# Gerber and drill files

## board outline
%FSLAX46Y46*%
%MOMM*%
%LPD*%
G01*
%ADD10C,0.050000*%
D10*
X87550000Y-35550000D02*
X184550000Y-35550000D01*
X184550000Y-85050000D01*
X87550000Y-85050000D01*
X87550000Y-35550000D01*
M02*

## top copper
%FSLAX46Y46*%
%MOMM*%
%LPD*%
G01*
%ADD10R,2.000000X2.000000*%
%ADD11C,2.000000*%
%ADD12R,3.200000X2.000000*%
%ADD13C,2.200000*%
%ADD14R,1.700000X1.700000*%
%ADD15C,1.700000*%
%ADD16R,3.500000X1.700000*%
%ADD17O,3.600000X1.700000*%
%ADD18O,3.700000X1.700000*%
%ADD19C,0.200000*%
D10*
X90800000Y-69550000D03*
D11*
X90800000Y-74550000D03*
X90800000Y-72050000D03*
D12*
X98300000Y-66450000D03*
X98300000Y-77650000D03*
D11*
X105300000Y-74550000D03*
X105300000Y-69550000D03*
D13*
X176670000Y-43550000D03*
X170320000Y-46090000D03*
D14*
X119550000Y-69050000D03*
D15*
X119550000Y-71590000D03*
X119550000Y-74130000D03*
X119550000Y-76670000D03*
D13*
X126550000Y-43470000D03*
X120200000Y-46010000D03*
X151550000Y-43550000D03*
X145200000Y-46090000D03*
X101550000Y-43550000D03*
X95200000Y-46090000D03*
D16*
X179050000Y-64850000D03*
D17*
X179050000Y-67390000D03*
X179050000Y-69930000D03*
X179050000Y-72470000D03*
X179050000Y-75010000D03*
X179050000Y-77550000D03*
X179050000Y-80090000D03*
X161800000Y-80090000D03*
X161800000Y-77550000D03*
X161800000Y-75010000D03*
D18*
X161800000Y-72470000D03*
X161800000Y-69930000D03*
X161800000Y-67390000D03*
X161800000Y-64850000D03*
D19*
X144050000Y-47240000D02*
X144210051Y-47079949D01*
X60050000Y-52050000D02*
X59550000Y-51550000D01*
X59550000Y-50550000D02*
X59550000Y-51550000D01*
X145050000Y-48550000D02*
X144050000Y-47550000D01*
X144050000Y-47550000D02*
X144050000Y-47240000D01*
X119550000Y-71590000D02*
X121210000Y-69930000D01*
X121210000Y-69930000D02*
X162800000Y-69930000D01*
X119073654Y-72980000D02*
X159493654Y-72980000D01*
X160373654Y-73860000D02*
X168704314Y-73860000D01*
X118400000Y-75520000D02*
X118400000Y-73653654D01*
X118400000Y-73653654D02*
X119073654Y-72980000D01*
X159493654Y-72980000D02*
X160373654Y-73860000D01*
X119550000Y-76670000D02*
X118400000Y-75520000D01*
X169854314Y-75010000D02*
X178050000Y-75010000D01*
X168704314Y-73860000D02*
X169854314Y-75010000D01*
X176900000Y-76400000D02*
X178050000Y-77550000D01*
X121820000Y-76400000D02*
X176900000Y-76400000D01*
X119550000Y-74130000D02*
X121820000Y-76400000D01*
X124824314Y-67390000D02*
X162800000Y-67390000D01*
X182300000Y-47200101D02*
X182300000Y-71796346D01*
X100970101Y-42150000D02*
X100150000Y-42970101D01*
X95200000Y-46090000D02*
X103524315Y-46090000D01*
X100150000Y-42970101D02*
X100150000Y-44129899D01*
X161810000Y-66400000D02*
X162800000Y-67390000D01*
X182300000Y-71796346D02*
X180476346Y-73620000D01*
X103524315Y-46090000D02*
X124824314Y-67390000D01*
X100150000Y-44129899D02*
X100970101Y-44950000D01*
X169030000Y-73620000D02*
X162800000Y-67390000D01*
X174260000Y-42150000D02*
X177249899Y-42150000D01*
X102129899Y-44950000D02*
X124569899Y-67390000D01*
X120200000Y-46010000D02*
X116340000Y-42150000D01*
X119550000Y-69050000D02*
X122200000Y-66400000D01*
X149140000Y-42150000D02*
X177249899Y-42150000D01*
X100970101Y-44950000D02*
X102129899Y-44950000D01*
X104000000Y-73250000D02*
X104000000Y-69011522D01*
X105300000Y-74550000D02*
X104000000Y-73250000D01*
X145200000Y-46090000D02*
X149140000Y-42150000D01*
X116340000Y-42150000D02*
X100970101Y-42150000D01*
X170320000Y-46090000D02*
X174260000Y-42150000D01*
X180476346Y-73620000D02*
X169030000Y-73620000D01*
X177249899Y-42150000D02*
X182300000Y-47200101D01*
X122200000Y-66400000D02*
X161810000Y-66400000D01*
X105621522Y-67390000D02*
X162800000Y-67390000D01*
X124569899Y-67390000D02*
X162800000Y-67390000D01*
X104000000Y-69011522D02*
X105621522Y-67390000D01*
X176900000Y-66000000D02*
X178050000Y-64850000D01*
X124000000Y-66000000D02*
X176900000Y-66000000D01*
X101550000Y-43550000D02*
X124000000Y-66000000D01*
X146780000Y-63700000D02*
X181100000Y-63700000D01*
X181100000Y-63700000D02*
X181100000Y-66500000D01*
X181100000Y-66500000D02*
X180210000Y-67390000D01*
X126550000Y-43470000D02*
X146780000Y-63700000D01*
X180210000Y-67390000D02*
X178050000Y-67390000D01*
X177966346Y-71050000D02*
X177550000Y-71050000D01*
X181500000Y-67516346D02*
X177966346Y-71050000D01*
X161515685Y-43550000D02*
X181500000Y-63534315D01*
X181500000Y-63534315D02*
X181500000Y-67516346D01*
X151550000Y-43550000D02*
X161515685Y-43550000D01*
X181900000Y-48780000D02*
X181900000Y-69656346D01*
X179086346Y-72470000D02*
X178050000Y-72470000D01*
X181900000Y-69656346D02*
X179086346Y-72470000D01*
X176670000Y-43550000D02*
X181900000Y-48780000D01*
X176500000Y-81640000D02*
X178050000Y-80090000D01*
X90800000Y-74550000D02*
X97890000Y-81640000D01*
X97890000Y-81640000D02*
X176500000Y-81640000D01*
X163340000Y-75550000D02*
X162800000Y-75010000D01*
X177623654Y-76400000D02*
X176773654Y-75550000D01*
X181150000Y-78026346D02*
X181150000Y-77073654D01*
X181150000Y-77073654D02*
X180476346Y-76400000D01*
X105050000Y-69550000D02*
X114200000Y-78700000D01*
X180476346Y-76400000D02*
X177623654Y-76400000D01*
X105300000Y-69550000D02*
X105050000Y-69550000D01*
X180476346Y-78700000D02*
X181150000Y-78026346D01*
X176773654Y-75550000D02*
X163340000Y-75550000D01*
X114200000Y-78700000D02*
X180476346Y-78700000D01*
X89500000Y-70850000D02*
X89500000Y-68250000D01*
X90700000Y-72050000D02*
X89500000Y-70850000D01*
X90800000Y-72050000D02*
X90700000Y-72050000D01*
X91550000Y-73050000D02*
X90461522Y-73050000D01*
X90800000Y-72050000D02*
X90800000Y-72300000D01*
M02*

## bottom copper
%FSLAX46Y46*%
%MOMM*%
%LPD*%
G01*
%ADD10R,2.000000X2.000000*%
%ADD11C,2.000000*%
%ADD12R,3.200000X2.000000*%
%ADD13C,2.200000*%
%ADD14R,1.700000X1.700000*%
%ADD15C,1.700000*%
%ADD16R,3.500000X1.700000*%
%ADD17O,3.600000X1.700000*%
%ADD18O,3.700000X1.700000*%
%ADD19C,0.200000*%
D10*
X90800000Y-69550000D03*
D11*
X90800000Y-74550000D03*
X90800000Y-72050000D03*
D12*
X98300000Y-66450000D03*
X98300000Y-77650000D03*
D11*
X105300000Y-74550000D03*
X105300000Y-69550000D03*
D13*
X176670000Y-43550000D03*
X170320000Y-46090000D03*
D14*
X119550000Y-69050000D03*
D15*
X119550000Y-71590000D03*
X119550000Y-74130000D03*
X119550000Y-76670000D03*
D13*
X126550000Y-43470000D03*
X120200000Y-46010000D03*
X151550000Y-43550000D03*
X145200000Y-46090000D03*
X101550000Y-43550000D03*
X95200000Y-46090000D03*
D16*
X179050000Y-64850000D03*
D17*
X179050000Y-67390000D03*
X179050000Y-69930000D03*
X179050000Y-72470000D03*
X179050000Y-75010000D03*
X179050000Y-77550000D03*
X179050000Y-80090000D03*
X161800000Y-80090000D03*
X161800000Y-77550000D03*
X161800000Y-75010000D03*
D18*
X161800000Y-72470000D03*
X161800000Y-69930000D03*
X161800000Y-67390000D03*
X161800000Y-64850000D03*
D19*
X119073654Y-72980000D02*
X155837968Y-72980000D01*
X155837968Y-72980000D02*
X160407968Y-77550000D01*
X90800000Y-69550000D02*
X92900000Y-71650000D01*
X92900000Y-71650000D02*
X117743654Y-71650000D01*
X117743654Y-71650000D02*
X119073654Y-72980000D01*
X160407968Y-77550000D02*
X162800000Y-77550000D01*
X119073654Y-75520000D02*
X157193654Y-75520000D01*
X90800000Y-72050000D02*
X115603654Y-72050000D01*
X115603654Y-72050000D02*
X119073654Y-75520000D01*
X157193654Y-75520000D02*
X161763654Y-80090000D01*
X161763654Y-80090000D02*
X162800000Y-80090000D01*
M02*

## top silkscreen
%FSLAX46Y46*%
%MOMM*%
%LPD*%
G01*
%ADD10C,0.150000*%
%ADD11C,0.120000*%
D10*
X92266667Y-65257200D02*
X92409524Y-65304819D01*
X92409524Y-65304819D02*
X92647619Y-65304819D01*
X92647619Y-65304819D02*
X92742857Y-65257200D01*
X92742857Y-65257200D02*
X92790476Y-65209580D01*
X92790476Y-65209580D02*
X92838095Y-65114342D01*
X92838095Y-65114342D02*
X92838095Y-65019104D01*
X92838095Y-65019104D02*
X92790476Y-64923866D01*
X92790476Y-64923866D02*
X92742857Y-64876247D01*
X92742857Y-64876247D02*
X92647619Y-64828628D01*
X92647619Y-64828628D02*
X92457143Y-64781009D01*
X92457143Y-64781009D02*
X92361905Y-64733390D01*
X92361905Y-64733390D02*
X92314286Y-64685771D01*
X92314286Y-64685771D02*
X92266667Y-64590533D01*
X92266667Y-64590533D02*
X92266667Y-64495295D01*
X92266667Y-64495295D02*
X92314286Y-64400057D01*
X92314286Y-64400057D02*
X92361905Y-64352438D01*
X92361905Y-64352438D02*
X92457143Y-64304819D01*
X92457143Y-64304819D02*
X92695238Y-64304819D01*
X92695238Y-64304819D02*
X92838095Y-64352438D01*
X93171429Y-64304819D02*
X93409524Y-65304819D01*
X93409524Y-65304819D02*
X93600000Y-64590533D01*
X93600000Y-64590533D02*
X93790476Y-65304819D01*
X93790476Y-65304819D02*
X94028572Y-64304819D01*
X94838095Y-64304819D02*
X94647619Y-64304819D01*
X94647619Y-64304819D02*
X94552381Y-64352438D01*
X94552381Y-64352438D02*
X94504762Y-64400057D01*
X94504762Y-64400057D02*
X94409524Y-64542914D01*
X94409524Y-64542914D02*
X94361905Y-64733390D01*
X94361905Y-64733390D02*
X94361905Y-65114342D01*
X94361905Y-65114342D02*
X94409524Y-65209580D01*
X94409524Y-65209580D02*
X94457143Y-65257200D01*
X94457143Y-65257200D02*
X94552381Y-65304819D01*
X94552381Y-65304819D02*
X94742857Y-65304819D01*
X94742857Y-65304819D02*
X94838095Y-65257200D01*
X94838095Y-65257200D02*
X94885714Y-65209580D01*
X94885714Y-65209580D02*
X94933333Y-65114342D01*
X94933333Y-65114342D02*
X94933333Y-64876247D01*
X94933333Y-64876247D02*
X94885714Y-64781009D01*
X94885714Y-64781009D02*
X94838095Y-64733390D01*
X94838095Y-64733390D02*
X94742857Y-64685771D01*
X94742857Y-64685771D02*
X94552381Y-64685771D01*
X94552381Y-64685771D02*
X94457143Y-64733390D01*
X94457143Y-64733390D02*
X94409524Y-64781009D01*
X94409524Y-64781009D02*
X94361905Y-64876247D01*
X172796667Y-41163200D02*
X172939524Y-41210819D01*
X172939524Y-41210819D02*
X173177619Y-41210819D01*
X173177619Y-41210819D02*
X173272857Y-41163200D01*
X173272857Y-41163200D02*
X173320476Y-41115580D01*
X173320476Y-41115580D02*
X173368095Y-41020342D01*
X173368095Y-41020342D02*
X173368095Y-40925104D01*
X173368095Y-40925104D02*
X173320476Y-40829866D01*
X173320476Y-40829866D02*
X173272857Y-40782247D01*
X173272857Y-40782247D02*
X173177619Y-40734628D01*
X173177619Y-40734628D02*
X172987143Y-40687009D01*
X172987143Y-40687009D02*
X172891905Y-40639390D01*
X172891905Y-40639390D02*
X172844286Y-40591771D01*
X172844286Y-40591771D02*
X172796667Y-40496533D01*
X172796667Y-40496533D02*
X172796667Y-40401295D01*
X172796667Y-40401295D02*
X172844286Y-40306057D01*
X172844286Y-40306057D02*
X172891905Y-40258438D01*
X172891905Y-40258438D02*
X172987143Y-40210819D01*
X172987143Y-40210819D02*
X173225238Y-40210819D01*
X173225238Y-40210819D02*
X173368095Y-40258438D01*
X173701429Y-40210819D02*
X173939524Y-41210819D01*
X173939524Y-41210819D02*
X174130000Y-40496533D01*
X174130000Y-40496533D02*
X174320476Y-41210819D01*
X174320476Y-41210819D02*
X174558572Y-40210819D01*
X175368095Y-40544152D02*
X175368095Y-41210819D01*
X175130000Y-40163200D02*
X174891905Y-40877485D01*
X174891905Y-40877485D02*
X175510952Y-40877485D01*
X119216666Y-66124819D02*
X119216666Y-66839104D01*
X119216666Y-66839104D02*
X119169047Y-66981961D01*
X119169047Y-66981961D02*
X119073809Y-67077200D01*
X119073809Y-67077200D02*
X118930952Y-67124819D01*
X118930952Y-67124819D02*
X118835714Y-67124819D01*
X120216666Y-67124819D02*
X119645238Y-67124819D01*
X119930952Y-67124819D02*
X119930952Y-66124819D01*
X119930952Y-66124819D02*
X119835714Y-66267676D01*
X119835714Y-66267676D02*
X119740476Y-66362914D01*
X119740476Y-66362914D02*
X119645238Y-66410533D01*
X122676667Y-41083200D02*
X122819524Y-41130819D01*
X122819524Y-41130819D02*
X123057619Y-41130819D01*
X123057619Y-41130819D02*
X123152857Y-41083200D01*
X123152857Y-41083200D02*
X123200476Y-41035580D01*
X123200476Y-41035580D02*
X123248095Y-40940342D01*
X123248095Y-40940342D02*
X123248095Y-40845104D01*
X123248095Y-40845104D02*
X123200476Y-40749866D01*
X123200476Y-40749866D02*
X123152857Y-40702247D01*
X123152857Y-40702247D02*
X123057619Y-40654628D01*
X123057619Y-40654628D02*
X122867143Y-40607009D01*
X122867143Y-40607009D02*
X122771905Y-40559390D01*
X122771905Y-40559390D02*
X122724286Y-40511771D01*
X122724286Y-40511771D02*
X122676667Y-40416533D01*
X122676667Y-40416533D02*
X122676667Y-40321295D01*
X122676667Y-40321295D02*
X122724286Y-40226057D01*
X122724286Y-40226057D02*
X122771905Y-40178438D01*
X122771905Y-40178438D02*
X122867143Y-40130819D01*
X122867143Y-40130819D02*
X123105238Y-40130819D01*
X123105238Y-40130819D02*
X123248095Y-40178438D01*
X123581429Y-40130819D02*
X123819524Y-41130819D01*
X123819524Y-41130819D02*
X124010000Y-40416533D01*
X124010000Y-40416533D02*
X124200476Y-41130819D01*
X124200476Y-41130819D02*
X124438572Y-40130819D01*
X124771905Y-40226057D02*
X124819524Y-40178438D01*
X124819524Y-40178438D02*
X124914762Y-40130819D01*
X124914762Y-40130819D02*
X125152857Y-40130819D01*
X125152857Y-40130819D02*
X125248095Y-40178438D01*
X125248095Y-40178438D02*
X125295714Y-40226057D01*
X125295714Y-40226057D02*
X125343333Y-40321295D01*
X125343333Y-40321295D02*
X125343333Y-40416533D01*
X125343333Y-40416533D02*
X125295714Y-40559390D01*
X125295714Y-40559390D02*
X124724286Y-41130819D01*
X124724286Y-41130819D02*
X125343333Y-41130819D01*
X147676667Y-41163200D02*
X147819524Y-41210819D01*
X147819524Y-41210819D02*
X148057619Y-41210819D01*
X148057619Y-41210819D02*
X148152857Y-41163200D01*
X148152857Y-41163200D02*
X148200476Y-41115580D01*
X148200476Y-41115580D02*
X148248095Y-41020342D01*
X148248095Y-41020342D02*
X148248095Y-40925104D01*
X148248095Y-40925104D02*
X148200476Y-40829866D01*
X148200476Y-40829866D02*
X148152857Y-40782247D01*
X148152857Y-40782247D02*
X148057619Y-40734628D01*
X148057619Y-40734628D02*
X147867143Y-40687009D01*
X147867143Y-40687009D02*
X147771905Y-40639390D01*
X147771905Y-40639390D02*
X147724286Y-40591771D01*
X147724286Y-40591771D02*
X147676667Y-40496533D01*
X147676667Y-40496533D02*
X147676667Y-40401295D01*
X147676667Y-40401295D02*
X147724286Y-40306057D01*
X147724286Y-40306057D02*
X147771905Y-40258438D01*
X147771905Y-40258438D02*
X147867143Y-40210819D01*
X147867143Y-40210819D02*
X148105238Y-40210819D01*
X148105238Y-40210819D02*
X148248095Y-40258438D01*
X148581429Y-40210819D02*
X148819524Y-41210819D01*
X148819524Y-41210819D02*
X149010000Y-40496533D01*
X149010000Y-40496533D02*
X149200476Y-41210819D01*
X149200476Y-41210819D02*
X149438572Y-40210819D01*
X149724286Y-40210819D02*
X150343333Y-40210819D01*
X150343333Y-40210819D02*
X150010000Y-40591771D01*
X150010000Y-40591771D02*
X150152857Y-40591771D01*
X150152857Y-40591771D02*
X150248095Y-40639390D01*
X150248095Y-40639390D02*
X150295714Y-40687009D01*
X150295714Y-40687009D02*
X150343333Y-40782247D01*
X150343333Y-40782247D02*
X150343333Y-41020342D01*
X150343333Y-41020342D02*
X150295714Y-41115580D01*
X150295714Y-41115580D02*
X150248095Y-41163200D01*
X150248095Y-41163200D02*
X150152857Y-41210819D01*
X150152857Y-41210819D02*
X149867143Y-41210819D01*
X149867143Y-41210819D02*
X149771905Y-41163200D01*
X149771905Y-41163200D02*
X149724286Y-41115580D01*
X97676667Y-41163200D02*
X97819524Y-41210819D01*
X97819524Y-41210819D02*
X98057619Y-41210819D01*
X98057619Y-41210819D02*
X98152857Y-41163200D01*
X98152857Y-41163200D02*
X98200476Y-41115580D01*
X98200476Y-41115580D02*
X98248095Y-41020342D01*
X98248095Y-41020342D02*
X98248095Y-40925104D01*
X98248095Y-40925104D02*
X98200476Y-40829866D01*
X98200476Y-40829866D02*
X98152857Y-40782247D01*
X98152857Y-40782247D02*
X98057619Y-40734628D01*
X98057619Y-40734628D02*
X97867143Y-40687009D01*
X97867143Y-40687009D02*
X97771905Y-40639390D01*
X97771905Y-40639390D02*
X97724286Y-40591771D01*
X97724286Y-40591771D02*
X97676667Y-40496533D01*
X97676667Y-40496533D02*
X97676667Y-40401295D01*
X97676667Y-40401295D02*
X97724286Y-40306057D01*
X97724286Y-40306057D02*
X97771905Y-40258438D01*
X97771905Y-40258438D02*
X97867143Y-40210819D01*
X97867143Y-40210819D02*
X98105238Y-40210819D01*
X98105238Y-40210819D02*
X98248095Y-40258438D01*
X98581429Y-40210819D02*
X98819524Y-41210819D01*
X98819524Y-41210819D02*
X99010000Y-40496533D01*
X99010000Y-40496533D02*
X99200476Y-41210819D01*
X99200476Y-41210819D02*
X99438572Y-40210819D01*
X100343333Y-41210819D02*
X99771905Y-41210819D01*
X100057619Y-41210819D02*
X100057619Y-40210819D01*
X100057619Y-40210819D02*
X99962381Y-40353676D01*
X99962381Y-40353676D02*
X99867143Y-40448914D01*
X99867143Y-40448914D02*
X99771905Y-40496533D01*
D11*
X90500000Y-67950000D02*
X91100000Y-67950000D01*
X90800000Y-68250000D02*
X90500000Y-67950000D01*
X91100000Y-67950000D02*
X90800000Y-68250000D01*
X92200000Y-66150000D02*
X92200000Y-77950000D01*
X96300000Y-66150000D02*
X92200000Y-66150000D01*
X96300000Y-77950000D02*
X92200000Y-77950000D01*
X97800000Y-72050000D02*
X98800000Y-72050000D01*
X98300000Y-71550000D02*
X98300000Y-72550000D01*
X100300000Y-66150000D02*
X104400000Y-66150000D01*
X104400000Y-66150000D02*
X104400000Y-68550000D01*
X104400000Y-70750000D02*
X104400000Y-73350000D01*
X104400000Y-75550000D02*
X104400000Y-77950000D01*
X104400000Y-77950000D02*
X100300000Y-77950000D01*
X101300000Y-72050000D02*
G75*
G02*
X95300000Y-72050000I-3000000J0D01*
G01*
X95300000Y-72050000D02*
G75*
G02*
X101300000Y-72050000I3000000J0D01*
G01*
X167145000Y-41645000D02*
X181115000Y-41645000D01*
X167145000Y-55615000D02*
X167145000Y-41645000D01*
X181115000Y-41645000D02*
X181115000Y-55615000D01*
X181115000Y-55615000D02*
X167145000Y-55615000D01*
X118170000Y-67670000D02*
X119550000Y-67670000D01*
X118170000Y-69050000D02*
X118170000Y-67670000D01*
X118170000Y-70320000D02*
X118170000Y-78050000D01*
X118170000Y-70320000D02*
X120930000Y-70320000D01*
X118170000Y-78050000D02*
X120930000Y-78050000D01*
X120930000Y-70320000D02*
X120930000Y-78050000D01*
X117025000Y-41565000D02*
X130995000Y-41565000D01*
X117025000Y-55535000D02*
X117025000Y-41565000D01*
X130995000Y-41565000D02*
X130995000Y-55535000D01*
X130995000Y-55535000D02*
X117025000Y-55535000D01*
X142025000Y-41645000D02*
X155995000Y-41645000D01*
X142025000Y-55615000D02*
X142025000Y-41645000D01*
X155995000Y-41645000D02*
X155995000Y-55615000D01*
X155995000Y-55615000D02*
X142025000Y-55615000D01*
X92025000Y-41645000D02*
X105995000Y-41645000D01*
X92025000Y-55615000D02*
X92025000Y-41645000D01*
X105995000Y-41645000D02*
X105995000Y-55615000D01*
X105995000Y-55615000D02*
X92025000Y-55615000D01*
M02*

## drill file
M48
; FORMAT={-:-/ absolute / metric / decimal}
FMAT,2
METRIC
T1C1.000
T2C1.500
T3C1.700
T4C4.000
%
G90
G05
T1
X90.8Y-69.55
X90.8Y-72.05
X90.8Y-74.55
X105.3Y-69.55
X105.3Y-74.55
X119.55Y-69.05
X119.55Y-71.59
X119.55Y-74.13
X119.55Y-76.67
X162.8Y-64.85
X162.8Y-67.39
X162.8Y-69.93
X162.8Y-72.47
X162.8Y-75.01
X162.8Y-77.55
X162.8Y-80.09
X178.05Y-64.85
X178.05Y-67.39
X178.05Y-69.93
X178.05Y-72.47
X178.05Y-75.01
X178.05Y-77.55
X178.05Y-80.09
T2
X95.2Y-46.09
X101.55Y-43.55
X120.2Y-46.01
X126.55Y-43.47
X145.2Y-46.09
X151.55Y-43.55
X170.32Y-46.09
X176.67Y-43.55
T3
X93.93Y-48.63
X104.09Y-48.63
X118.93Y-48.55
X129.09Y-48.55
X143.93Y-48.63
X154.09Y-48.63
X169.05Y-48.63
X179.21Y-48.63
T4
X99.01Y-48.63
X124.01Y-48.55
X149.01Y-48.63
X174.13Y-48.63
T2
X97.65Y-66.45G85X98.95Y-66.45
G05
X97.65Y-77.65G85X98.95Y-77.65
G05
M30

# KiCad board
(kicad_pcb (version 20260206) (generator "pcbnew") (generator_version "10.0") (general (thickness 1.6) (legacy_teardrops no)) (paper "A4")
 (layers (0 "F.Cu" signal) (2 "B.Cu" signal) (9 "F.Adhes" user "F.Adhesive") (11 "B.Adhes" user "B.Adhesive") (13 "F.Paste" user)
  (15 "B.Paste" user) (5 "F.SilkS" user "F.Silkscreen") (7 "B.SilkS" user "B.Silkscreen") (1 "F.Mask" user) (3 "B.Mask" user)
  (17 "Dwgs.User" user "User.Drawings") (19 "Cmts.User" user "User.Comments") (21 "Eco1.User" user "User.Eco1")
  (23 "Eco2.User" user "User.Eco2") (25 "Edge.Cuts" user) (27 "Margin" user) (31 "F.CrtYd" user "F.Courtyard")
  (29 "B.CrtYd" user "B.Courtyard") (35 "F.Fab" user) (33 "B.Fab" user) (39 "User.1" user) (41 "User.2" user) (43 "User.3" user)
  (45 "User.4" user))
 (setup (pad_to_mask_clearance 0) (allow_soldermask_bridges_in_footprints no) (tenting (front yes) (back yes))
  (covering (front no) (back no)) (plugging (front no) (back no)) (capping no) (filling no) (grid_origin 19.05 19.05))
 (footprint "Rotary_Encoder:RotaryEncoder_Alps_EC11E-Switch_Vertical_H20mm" (layer "F.Cu") (at 90.8 69.55)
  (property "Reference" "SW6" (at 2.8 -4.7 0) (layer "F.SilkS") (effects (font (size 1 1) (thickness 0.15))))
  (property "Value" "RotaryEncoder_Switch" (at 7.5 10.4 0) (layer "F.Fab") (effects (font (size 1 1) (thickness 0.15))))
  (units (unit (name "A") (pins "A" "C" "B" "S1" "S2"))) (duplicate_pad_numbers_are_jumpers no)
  (fp_line (start -0.3 -1.6) (end 0.3 -1.6) (stroke (width 0.12) (type solid)) (layer "F.SilkS"))
  (fp_line (start 0 -1.3) (end -0.3 -1.6) (stroke (width 0.12) (type solid)) (layer "F.SilkS"))
  (fp_line (start 0.3 -1.6) (end 0 -1.3) (stroke (width 0.12) (type solid)) (layer "F.SilkS"))
  (fp_line (start 1.4 -3.4) (end 1.4 8.4) (stroke (width 0.12) (type solid)) (layer "F.SilkS"))
  (fp_line (start 5.5 -3.4) (end 1.4 -3.4) (stroke (width 0.12) (type solid)) (layer "F.SilkS"))
  (fp_line (start 5.5 8.4) (end 1.4 8.4) (stroke (width 0.12) (type solid)) (layer "F.SilkS"))
  (fp_line (start 7 2.5) (end 8 2.5) (stroke (width 0.12) (type solid)) (layer "F.SilkS"))
  (fp_line (start 7.5 2) (end 7.5 3) (stroke (width 0.12) (type solid)) (layer "F.SilkS"))
  (fp_line (start 9.5 -3.4) (end 13.6 -3.4) (stroke (width 0.12) (type solid)) (layer "F.SilkS"))
  (fp_line (start 13.6 -3.4) (end 13.6 -1) (stroke (width 0.12) (type solid)) (layer "F.SilkS"))
  (fp_line (start 13.6 1.2) (end 13.6 3.8) (stroke (width 0.12) (type solid)) (layer "F.SilkS"))
  (fp_line (start 13.6 6) (end 13.6 8.4) (stroke (width 0.12) (type solid)) (layer "F.SilkS"))
  (fp_line (start 13.6 8.4) (end 9.5 8.4) (stroke (width 0.12) (type solid)) (layer "F.SilkS"))
  (fp_circle (center 7.5 2.5) (end 10.5 2.5) (stroke (width 0.12) (type solid)) (fill no) (layer "F.SilkS"))
  (pad "A" thru_hole rect (at 0 0) (size 2 2) (drill 1) (layers "*.Cu" "*.Mask") (remove_unused_layers no) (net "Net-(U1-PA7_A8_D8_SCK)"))
  (pad "B" thru_hole circle (at 0 5) (size 2 2) (drill 1) (layers "*.Cu" "*.Mask") (remove_unused_layers no) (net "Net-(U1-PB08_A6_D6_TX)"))
  (pad "C" thru_hole circle (at 0 2.5) (size 2 2) (drill 1) (layers "*.Cu" "*.Mask") (remove_unused_layers no)
   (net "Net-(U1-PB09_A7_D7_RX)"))
  (pad "MP" thru_hole rect (at 7.5 -3.1) (size 3.2 2) (drill oval 2.8 1.5) (layers "*.Cu" "*.Mask") (remove_unused_layers no))
  (pad "MP" thru_hole rect (at 7.5 8.1) (size 3.2 2) (drill oval 2.8 1.5) (layers "*.Cu" "*.Mask") (remove_unused_layers no))
  (pad "S1" thru_hole circle (at 14.5 5) (size 2 2) (drill 1) (layers "*.Cu" "*.Mask") (remove_unused_layers no) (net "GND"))
  (pad "S2" thru_hole circle (at 14.5 0) (size 2 2) (drill 1) (layers "*.Cu" "*.Mask") (remove_unused_layers no)
   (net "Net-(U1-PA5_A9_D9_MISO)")))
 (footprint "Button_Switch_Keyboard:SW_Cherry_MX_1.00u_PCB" (layer "F.Cu") (at 176.67 43.55)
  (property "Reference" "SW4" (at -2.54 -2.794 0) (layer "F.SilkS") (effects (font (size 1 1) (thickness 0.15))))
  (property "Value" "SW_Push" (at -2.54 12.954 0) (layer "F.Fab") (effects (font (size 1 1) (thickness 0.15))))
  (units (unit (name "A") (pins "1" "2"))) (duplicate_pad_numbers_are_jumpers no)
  (fp_line (start -9.525 -1.905) (end 4.445 -1.905) (stroke (width 0.12) (type solid)) (layer "F.SilkS"))
  (fp_line (start -9.525 12.065) (end -9.525 -1.905) (stroke (width 0.12) (type solid)) (layer "F.SilkS"))
  (fp_line (start 4.445 -1.905) (end 4.445 12.065) (stroke (width 0.12) (type solid)) (layer "F.SilkS"))
  (fp_line (start 4.445 12.065) (end -9.525 12.065) (stroke (width 0.12) (type solid)) (layer "F.SilkS"))
  (pad "" np_thru_hole circle (at -7.62 5.08) (size 1.7 1.7) (drill 1.7) (layers "*.Cu" "*.Mask"))
  (pad "" np_thru_hole circle (at -2.54 5.08) (size 4 4) (drill 4) (layers "*.Cu" "*.Mask"))
  (pad "" np_thru_hole circle (at 2.54 5.08) (size 1.7 1.7) (drill 1.7) (layers "*.Cu" "*.Mask"))
  (pad "1" thru_hole circle (at 0 0) (size 2.2 2.2) (drill 1.5) (layers "*.Cu" "*.Mask") (remove_unused_layers no)
   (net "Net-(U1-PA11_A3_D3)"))
  (pad "2" thru_hole circle (at -6.35 2.54) (size 2.2 2.2) (drill 1.5) (layers "*.Cu" "*.Mask") (remove_unused_layers no) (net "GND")))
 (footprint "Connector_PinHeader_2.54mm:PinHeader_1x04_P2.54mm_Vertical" (layer "F.Cu") (at 119.55 69.05)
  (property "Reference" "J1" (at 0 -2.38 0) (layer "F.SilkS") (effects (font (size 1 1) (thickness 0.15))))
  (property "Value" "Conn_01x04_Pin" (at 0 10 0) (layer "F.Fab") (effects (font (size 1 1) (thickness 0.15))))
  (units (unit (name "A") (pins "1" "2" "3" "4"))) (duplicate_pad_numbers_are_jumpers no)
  (fp_line (start -1.38 -1.38) (end 0 -1.38) (stroke (width 0.12) (type solid)) (layer "F.SilkS"))
  (fp_line (start -1.38 0) (end -1.38 -1.38) (stroke (width 0.12) (type solid)) (layer "F.SilkS"))
  (fp_line (start -1.38 1.27) (end -1.38 9) (stroke (width 0.12) (type solid)) (layer "F.SilkS"))
  (fp_line (start -1.38 1.27) (end 1.38 1.27) (stroke (width 0.12) (type solid)) (layer "F.SilkS"))
  (fp_line (start -1.38 9) (end 1.38 9) (stroke (width 0.12) (type solid)) (layer "F.SilkS"))
  (fp_line (start 1.38 1.27) (end 1.38 9) (stroke (width 0.12) (type solid)) (layer "F.SilkS"))
  (pad "1" thru_hole rect (at 0 0) (size 1.7 1.7) (drill 1) (layers "*.Cu" "*.Mask") (remove_unused_layers no) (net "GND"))
  (pad "2" thru_hole circle (at 0 2.54) (size 1.7 1.7) (drill 1) (layers "*.Cu" "*.Mask") (remove_unused_layers no) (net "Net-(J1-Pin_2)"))
  (pad "3" thru_hole circle (at 0 5.08) (size 1.7 1.7) (drill 1) (layers "*.Cu" "*.Mask") (remove_unused_layers no) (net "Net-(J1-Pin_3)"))
  (pad "4" thru_hole circle (at 0 7.62) (size 1.7 1.7) (drill 1) (layers "*.Cu" "*.Mask") (remove_unused_layers no) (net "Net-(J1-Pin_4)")))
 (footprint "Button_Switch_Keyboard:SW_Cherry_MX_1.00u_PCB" (layer "F.Cu") (at 126.55 43.47)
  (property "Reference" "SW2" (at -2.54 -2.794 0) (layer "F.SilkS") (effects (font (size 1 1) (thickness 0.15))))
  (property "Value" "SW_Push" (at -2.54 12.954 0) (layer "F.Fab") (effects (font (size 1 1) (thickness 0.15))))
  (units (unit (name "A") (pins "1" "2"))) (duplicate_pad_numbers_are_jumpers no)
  (fp_line (start -9.525 -1.905) (end 4.445 -1.905) (stroke (width 0.12) (type solid)) (layer "F.SilkS"))
  (fp_line (start -9.525 12.065) (end -9.525 -1.905) (stroke (width 0.12) (type solid)) (layer "F.SilkS"))
  (fp_line (start 4.445 -1.905) (end 4.445 12.065) (stroke (width 0.12) (type solid)) (layer "F.SilkS"))
  (fp_line (start 4.445 12.065) (end -9.525 12.065) (stroke (width 0.12) (type solid)) (layer "F.SilkS"))
  (pad "" np_thru_hole circle (at -7.62 5.08) (size 1.7 1.7) (drill 1.7) (layers "*.Cu" "*.Mask"))
  (pad "" np_thru_hole circle (at -2.54 5.08) (size 4 4) (drill 4) (layers "*.Cu" "*.Mask"))
  (pad "" np_thru_hole circle (at 2.54 5.08) (size 1.7 1.7) (drill 1.7) (layers "*.Cu" "*.Mask"))
  (pad "1" thru_hole circle (at 0 0) (size 2.2 2.2) (drill 1.5) (layers "*.Cu" "*.Mask") (remove_unused_layers no)
   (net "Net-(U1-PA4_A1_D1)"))
  (pad "2" thru_hole circle (at -6.35 2.54) (size 2.2 2.2) (drill 1.5) (layers "*.Cu" "*.Mask") (remove_unused_layers no) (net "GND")))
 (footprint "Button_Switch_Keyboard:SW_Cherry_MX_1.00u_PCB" (layer "F.Cu") (at 151.55 43.55)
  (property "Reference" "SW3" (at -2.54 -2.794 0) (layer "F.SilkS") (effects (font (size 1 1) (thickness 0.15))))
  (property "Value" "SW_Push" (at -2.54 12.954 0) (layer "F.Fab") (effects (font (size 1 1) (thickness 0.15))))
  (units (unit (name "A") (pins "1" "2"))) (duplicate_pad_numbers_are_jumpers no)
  (fp_line (start -9.525 -1.905) (end 4.445 -1.905) (stroke (width 0.12) (type solid)) (layer "F.SilkS"))
  (fp_line (start -9.525 12.065) (end -9.525 -1.905) (stroke (width 0.12) (type solid)) (layer "F.SilkS"))
  (fp_line (start 4.445 -1.905) (end 4.445 12.065) (stroke (width 0.12) (type solid)) (layer "F.SilkS"))
  (fp_line (start 4.445 12.065) (end -9.525 12.065) (stroke (width 0.12) (type solid)) (layer "F.SilkS"))
  (pad "" np_thru_hole circle (at -7.62 5.08) (size 1.7 1.7) (drill 1.7) (layers "*.Cu" "*.Mask"))
  (pad "" np_thru_hole circle (at -2.54 5.08) (size 4 4) (drill 4) (layers "*.Cu" "*.Mask"))
  (pad "" np_thru_hole circle (at 2.54 5.08) (size 1.7 1.7) (drill 1.7) (layers "*.Cu" "*.Mask"))
  (pad "1" thru_hole circle (at 0 0) (size 2.2 2.2) (drill 1.5) (layers "*.Cu" "*.Mask") (remove_unused_layers no)
   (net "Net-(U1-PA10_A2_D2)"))
  (pad "2" thru_hole circle (at -6.35 2.54) (size 2.2 2.2) (drill 1.5) (layers "*.Cu" "*.Mask") (remove_unused_layers no) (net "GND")))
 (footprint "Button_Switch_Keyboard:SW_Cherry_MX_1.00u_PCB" (layer "F.Cu") (at 101.55 43.55)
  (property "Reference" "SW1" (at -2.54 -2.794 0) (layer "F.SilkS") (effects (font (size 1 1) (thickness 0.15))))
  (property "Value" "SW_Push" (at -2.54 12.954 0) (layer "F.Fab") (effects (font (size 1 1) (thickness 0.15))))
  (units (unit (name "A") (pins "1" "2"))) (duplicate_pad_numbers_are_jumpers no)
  (fp_line (start -9.525 -1.905) (end 4.445 -1.905) (stroke (width 0.12) (type solid)) (layer "F.SilkS"))
  (fp_line (start -9.525 12.065) (end -9.525 -1.905) (stroke (width 0.12) (type solid)) (layer "F.SilkS"))
  (fp_line (start 4.445 -1.905) (end 4.445 12.065) (stroke (width 0.12) (type solid)) (layer "F.SilkS"))
  (fp_line (start 4.445 12.065) (end -9.525 12.065) (stroke (width 0.12) (type solid)) (layer "F.SilkS"))
  (pad "" np_thru_hole circle (at -7.62 5.08) (size 1.7 1.7) (drill 1.7) (layers "*.Cu" "*.Mask"))
  (pad "" np_thru_hole circle (at -2.54 5.08) (size 4 4) (drill 4) (layers "*.Cu" "*.Mask"))
  (pad "" np_thru_hole circle (at 2.54 5.08) (size 1.7 1.7) (drill 1.7) (layers "*.Cu" "*.Mask"))
  (pad "1" thru_hole circle (at 0 0) (size 2.2 2.2) (drill 1.5) (layers "*.Cu" "*.Mask") (remove_unused_layers no)
   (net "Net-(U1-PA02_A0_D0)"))
  (pad "2" thru_hole circle (at -6.35 2.54) (size 2.2 2.2) (drill 1.5) (layers "*.Cu" "*.Mask") (remove_unused_layers no) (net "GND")))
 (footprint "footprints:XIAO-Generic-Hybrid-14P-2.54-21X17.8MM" (layer "B.Cu") (at 170.425 72.47 180)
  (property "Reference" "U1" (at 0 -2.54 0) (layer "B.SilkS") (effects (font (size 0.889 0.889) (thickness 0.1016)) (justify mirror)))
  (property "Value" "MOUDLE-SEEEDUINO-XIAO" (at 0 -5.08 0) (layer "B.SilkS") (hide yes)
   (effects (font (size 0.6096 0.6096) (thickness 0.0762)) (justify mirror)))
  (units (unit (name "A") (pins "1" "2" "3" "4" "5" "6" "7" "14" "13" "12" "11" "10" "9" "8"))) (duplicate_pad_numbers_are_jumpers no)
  (pad "1" thru_hole rect (at -7.625 7.62 180) (size 3.5 1.7) (drill 1 (offset -1 0)) (layers "*.Cu" "*.Mask") (remove_unused_layers no)
   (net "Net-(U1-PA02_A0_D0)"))
  (pad "2" thru_hole oval (at -7.625 5.08 180) (size 3.6 1.7) (drill 1 (offset -1 0)) (layers "*.Cu" "*.Mask") (remove_unused_layers no)
   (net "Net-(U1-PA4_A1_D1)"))
  (pad "3" thru_hole oval (at -7.625 2.54 180) (size 3.6 1.7) (drill 1 (offset -1 0)) (layers "*.Cu" "*.Mask") (remove_unused_layers no)
   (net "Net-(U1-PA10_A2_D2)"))
  (pad "4" thru_hole oval (at -7.625 0 180) (size 3.6 1.7) (drill 1 (offset -1 0)) (layers "*.Cu" "*.Mask") (remove_unused_layers no)
   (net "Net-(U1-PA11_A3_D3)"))
  (pad "5" thru_hole oval (at -7.625 -2.54 180) (size 3.6 1.7) (drill 1 (offset -1 0)) (layers "*.Cu" "*.Mask") (remove_unused_layers no)
   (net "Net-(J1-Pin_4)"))
  (pad "6" thru_hole oval (at -7.625 -5.08) (size 3.6 1.7) (drill 1 (offset 1 0)) (layers "*.Cu" "*.Mask") (remove_unused_layers no)
   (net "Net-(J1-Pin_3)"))
  (pad "7" thru_hole oval (at -7.625 -7.62 180) (size 3.6 1.7) (drill 1 (offset -1 0)) (layers "*.Cu" "*.Mask") (remove_unused_layers no)
   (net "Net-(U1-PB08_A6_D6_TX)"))
  (pad "8" thru_hole oval (at 7.625 -7.62 180) (size 3.6 1.7) (drill 1 (offset 1 0)) (layers "*.Cu" "*.Mask") (remove_unused_layers no)
   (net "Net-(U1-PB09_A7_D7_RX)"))
  (pad "9" thru_hole oval (at 7.625 -5.08 180) (size 3.6 1.7) (drill 1 (offset 1 0)) (layers "*.Cu" "*.Mask") (remove_unused_layers no)
   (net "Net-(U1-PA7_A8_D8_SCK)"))
  (pad "10" thru_hole oval (at 7.625 -2.54 180) (size 3.6 1.7) (drill 1 (offset 1 0)) (layers "*.Cu" "*.Mask") (remove_unused_layers no)
   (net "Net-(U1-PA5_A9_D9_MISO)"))
  (pad "11" thru_hole oval (at 7.625 0 180) (size 3.7 1.7) (drill 1 (offset 1 0)) (layers "*.Cu" "*.Mask") (remove_unused_layers no)
   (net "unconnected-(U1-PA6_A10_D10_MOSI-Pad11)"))
  (pad "12" thru_hole oval (at 7.625 2.54 180) (size 3.7 1.7) (drill 1 (offset 1 0)) (layers "*.Cu" "*.Mask") (remove_unused_layers no)
   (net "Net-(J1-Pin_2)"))
  (pad "13" thru_hole oval (at 7.625 5.08 180) (size 3.7 1.7) (drill 1 (offset 1 0)) (layers "*.Cu" "*.Mask") (remove_unused_layers no)
   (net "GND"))
  (pad "14" thru_hole oval (at 7.625 7.62 180) (size 3.7 1.7) (drill 1 (offset 1 0)) (layers "*.Cu" "*.Mask") (remove_unused_layers no)
   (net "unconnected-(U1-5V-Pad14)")))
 (gr_rect (start 87.55 35.55) (end 184.55 85.05) (stroke (width 0.05) (type solid)) (fill no) (layer "Edge.Cuts"))
 (segment (start 144.05 47.24) (end 144.210051 47.079949) (width 0.2) (layer "F.Cu") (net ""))
 (segment (start 60.05 52.05) (end 59.55 51.55) (width 0.2) (layer "F.Cu") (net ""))
 (segment (start 59.55 50.55) (end 59.55 51.55) (width 0.2) (layer "F.Cu") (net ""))
 (segment (start 145.05 48.55) (end 144.05 47.55) (width 0.2) (layer "F.Cu") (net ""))
 (segment (start 144.05 47.55) (end 144.05 47.24) (width 0.2) (layer "F.Cu") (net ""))
 (segment (start 119.55 71.59) (end 121.21 69.93) (width 0.2) (layer "F.Cu") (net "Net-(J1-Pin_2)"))
 (segment (start 121.21 69.93) (end 162.8 69.93) (width 0.2) (layer "F.Cu") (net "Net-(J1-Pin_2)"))
 (segment (start 119.073654 72.98) (end 159.493654 72.98) (width 0.2) (layer "F.Cu") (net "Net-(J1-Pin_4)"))
 (segment (start 160.373654 73.86) (end 168.704314 73.86) (width 0.2) (layer "F.Cu") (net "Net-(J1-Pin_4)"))
 (segment (start 118.4 75.52) (end 118.4 73.653654) (width 0.2) (layer "F.Cu") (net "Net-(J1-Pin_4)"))
 (segment (start 118.4 73.653654) (end 119.073654 72.98) (width 0.2) (layer "F.Cu") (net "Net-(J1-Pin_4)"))
 (segment (start 159.493654 72.98) (end 160.373654 73.86) (width 0.2) (layer "F.Cu") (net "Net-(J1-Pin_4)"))
 (segment (start 119.55 76.67) (end 118.4 75.52) (width 0.2) (layer "F.Cu") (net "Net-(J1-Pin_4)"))
 (segment (start 169.854314 75.01) (end 178.05 75.01) (width 0.2) (layer "F.Cu") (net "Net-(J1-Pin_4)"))
 (segment (start 168.704314 73.86) (end 169.854314 75.01) (width 0.2) (layer "F.Cu") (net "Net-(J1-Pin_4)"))
 (segment (start 176.9 76.4) (end 178.05 77.55) (width 0.2) (layer "F.Cu") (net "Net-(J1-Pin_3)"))
 (segment (start 121.82 76.4) (end 176.9 76.4) (width 0.2) (layer "F.Cu") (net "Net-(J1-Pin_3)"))
 (segment (start 119.55 74.13) (end 121.82 76.4) (width 0.2) (layer "F.Cu") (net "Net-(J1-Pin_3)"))
 (segment (start 124.824314 67.39) (end 162.8 67.39) (width 0.2) (layer "F.Cu") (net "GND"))
 (segment (start 182.3 47.200101) (end 182.3 71.796346) (width 0.2) (layer "F.Cu") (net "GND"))
 (segment (start 100.970101 42.15) (end 100.15 42.970101) (width 0.2) (layer "F.Cu") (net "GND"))
 (segment (start 95.2 46.09) (end 103.524315 46.09) (width 0.2) (layer "F.Cu") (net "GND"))
 (segment (start 100.15 42.970101) (end 100.15 44.129899) (width 0.2) (layer "F.Cu") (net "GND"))
 (segment (start 161.81 66.4) (end 162.8 67.39) (width 0.2) (layer "F.Cu") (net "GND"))
 (segment (start 182.3 71.796346) (end 180.476346 73.62) (width 0.2) (layer "F.Cu") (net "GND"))
 (segment (start 103.524315 46.09) (end 124.824314 67.39) (width 0.2) (layer "F.Cu") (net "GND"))
 (segment (start 100.15 44.129899) (end 100.970101 44.95) (width 0.2) (layer "F.Cu") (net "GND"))
 (segment (start 169.03 73.62) (end 162.8 67.39) (width 0.2) (layer "F.Cu") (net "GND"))
 (segment (start 174.26 42.15) (end 177.249899 42.15) (width 0.2) (layer "F.Cu") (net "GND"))
 (segment (start 102.129899 44.95) (end 124.569899 67.39) (width 0.2) (layer "F.Cu") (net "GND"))
 (segment (start 120.2 46.01) (end 116.34 42.15) (width 0.2) (layer "F.Cu") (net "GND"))
 (segment (start 119.55 69.05) (end 122.2 66.4) (width 0.2) (layer "F.Cu") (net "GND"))
 (segment (start 149.14 42.15) (end 177.249899 42.15) (width 0.2) (layer "F.Cu") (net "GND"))
 (segment (start 100.970101 44.95) (end 102.129899 44.95) (width 0.2) (layer "F.Cu") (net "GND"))
 (segment (start 104 73.25) (end 104 69.011522) (width 0.2) (layer "F.Cu") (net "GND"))
 (segment (start 105.3 74.55) (end 104 73.25) (width 0.2) (layer "F.Cu") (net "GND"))
 (segment (start 145.2 46.09) (end 149.14 42.15) (width 0.2) (layer "F.Cu") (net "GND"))
 (segment (start 116.34 42.15) (end 100.970101 42.15) (width 0.2) (layer "F.Cu") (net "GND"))
 (segment (start 170.32 46.09) (end 174.26 42.15) (width 0.2) (layer "F.Cu") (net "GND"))
 (segment (start 180.476346 73.62) (end 169.03 73.62) (width 0.2) (layer "F.Cu") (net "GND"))
 (segment (start 177.249899 42.15) (end 182.3 47.200101) (width 0.2) (layer "F.Cu") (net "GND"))
 (segment (start 122.2 66.4) (end 161.81 66.4) (width 0.2) (layer "F.Cu") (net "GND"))
 (segment (start 105.621522 67.39) (end 162.8 67.39) (width 0.2) (layer "F.Cu") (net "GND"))
 (segment (start 124.569899 67.39) (end 162.8 67.39) (width 0.2) (layer "F.Cu") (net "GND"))
 (segment (start 104 69.011522) (end 105.621522 67.39) (width 0.2) (layer "F.Cu") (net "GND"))
 (segment (start 176.9 66) (end 178.05 64.85) (width 0.2) (layer "F.Cu") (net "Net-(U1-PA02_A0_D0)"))
 (segment (start 124 66) (end 176.9 66) (width 0.2) (layer "F.Cu") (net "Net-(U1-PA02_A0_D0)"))
 (segment (start 101.55 43.55) (end 124 66) (width 0.2) (layer "F.Cu") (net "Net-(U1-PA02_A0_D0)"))
 (segment (start 146.78 63.7) (end 181.1 63.7) (width 0.2) (layer "F.Cu") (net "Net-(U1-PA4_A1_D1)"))
 (segment (start 181.1 63.7) (end 181.1 66.5) (width 0.2) (layer "F.Cu") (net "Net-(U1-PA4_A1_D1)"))
 (segment (start 181.1 66.5) (end 180.21 67.39) (width 0.2) (layer "F.Cu") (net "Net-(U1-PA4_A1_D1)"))
 (segment (start 126.55 43.47) (end 146.78 63.7) (width 0.2) (layer "F.Cu") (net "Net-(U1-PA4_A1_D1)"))
 (segment (start 180.21 67.39) (end 178.05 67.39) (width 0.2) (layer "F.Cu") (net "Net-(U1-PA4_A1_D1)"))
 (segment (start 177.966346 71.05) (end 177.55 71.05) (width 0.2) (layer "F.Cu") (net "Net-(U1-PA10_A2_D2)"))
 (segment (start 181.5 67.516346) (end 177.966346 71.05) (width 0.2) (layer "F.Cu") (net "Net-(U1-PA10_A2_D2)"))
 (segment (start 161.515685 43.55) (end 181.5 63.534315) (width 0.2) (layer "F.Cu") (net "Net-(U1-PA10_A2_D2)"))
 (segment (start 181.5 63.534315) (end 181.5 67.516346) (width 0.2) (layer "F.Cu") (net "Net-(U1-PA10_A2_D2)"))
 (segment (start 151.55 43.55) (end 161.515685 43.55) (width 0.2) (layer "F.Cu") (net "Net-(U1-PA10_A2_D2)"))
 (segment (start 181.9 48.78) (end 181.9 69.656346) (width 0.2) (layer "F.Cu") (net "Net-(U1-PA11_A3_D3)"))
 (segment (start 179.086346 72.47) (end 178.05 72.47) (width 0.2) (layer "F.Cu") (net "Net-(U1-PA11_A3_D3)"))
 (segment (start 181.9 69.656346) (end 179.086346 72.47) (width 0.2) (layer "F.Cu") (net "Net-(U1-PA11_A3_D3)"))
 (segment (start 176.67 43.55) (end 181.9 48.78) (width 0.2) (layer "F.Cu") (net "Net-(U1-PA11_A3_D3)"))
 (segment (start 176.5 81.64) (end 178.05 80.09) (width 0.2) (layer "F.Cu") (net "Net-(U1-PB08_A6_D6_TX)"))
 (segment (start 90.8 74.55) (end 97.89 81.64) (width 0.2) (layer "F.Cu") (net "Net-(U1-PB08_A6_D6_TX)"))
 (segment (start 97.89 81.64) (end 176.5 81.64) (width 0.2) (layer "F.Cu") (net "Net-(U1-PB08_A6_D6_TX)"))
 (segment (start 119.073654 72.98) (end 155.837968 72.98) (width 0.2) (layer "B.Cu") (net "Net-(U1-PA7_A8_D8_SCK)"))
 (segment (start 155.837968 72.98) (end 160.407968 77.55) (width 0.2) (layer "B.Cu") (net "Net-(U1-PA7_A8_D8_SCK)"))
 (segment (start 90.8 69.55) (end 92.9 71.65) (width 0.2) (layer "B.Cu") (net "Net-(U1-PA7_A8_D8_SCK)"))
 (segment (start 92.9 71.65) (end 117.743654 71.65) (width 0.2) (layer "B.Cu") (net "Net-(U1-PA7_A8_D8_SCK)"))
 (segment (start 117.743654 71.65) (end 119.073654 72.98) (width 0.2) (layer "B.Cu") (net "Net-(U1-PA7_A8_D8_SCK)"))
 (segment (start 160.407968 77.55) (end 162.8 77.55) (width 0.2) (layer "B.Cu") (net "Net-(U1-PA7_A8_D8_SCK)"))
 (segment (start 163.34 75.55) (end 162.8 75.01) (width 0.2) (layer "F.Cu") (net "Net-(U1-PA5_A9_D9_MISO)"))
 (segment (start 177.623654 76.4) (end 176.773654 75.55) (width 0.2) (layer "F.Cu") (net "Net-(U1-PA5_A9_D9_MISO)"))
 (segment (start 181.15 78.026346) (end 181.15 77.073654) (width 0.2) (layer "F.Cu") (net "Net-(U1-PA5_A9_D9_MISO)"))
 (segment (start 181.15 77.073654) (end 180.476346 76.4) (width 0.2) (layer "F.Cu") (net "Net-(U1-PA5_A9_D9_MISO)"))
 (segment (start 105.05 69.55) (end 114.2 78.7) (width 0.2) (layer "F.Cu") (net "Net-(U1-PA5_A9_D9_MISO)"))
 (segment (start 180.476346 76.4) (end 177.623654 76.4) (width 0.2) (layer "F.Cu") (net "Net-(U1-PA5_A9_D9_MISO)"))
 (segment (start 105.3 69.55) (end 105.05 69.55) (width 0.2) (layer "F.Cu") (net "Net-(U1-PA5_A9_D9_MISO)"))
 (segment (start 180.476346 78.7) (end 181.15 78.026346) (width 0.2) (layer "F.Cu") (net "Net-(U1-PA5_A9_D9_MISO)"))
 (segment (start 176.773654 75.55) (end 163.34 75.55) (width 0.2) (layer "F.Cu") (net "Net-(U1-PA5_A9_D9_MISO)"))
 (segment (start 114.2 78.7) (end 180.476346 78.7) (width 0.2) (layer "F.Cu") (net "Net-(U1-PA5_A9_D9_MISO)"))
 (segment (start 89.5 70.85) (end 89.5 68.25) (width 0.2) (layer "F.Cu") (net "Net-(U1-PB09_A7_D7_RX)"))
 (segment (start 90.7 72.05) (end 89.5 70.85) (width 0.2) (layer "F.Cu") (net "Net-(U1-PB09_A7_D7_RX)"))
 (segment (start 90.8 72.05) (end 90.7 72.05) (width 0.2) (layer "F.Cu") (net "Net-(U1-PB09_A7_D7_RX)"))
 (segment (start 91.55 73.05) (end 90.461522 73.05) (width 0.2) (layer "F.Cu") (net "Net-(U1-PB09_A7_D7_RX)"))
 (segment (start 90.8 72.05) (end 90.8 72.3) (width 0.2) (layer "F.Cu") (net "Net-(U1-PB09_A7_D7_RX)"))
 (segment (start 119.073654 75.52) (end 157.193654 75.52) (width 0.2) (layer "B.Cu") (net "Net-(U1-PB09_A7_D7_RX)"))
 (segment (start 90.8 72.05) (end 115.603654 72.05) (width 0.2) (layer "B.Cu") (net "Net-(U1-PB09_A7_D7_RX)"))
 (segment (start 115.603654 72.05) (end 119.073654 75.52) (width 0.2) (layer "B.Cu") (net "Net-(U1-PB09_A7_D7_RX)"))
 (segment (start 157.193654 75.52) (end 161.763654 80.09) (width 0.2) (layer "B.Cu") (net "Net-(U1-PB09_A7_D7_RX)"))
 (segment (start 161.763654 80.09) (end 162.8 80.09) (width 0.2) (layer "B.Cu") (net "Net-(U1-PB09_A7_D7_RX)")))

